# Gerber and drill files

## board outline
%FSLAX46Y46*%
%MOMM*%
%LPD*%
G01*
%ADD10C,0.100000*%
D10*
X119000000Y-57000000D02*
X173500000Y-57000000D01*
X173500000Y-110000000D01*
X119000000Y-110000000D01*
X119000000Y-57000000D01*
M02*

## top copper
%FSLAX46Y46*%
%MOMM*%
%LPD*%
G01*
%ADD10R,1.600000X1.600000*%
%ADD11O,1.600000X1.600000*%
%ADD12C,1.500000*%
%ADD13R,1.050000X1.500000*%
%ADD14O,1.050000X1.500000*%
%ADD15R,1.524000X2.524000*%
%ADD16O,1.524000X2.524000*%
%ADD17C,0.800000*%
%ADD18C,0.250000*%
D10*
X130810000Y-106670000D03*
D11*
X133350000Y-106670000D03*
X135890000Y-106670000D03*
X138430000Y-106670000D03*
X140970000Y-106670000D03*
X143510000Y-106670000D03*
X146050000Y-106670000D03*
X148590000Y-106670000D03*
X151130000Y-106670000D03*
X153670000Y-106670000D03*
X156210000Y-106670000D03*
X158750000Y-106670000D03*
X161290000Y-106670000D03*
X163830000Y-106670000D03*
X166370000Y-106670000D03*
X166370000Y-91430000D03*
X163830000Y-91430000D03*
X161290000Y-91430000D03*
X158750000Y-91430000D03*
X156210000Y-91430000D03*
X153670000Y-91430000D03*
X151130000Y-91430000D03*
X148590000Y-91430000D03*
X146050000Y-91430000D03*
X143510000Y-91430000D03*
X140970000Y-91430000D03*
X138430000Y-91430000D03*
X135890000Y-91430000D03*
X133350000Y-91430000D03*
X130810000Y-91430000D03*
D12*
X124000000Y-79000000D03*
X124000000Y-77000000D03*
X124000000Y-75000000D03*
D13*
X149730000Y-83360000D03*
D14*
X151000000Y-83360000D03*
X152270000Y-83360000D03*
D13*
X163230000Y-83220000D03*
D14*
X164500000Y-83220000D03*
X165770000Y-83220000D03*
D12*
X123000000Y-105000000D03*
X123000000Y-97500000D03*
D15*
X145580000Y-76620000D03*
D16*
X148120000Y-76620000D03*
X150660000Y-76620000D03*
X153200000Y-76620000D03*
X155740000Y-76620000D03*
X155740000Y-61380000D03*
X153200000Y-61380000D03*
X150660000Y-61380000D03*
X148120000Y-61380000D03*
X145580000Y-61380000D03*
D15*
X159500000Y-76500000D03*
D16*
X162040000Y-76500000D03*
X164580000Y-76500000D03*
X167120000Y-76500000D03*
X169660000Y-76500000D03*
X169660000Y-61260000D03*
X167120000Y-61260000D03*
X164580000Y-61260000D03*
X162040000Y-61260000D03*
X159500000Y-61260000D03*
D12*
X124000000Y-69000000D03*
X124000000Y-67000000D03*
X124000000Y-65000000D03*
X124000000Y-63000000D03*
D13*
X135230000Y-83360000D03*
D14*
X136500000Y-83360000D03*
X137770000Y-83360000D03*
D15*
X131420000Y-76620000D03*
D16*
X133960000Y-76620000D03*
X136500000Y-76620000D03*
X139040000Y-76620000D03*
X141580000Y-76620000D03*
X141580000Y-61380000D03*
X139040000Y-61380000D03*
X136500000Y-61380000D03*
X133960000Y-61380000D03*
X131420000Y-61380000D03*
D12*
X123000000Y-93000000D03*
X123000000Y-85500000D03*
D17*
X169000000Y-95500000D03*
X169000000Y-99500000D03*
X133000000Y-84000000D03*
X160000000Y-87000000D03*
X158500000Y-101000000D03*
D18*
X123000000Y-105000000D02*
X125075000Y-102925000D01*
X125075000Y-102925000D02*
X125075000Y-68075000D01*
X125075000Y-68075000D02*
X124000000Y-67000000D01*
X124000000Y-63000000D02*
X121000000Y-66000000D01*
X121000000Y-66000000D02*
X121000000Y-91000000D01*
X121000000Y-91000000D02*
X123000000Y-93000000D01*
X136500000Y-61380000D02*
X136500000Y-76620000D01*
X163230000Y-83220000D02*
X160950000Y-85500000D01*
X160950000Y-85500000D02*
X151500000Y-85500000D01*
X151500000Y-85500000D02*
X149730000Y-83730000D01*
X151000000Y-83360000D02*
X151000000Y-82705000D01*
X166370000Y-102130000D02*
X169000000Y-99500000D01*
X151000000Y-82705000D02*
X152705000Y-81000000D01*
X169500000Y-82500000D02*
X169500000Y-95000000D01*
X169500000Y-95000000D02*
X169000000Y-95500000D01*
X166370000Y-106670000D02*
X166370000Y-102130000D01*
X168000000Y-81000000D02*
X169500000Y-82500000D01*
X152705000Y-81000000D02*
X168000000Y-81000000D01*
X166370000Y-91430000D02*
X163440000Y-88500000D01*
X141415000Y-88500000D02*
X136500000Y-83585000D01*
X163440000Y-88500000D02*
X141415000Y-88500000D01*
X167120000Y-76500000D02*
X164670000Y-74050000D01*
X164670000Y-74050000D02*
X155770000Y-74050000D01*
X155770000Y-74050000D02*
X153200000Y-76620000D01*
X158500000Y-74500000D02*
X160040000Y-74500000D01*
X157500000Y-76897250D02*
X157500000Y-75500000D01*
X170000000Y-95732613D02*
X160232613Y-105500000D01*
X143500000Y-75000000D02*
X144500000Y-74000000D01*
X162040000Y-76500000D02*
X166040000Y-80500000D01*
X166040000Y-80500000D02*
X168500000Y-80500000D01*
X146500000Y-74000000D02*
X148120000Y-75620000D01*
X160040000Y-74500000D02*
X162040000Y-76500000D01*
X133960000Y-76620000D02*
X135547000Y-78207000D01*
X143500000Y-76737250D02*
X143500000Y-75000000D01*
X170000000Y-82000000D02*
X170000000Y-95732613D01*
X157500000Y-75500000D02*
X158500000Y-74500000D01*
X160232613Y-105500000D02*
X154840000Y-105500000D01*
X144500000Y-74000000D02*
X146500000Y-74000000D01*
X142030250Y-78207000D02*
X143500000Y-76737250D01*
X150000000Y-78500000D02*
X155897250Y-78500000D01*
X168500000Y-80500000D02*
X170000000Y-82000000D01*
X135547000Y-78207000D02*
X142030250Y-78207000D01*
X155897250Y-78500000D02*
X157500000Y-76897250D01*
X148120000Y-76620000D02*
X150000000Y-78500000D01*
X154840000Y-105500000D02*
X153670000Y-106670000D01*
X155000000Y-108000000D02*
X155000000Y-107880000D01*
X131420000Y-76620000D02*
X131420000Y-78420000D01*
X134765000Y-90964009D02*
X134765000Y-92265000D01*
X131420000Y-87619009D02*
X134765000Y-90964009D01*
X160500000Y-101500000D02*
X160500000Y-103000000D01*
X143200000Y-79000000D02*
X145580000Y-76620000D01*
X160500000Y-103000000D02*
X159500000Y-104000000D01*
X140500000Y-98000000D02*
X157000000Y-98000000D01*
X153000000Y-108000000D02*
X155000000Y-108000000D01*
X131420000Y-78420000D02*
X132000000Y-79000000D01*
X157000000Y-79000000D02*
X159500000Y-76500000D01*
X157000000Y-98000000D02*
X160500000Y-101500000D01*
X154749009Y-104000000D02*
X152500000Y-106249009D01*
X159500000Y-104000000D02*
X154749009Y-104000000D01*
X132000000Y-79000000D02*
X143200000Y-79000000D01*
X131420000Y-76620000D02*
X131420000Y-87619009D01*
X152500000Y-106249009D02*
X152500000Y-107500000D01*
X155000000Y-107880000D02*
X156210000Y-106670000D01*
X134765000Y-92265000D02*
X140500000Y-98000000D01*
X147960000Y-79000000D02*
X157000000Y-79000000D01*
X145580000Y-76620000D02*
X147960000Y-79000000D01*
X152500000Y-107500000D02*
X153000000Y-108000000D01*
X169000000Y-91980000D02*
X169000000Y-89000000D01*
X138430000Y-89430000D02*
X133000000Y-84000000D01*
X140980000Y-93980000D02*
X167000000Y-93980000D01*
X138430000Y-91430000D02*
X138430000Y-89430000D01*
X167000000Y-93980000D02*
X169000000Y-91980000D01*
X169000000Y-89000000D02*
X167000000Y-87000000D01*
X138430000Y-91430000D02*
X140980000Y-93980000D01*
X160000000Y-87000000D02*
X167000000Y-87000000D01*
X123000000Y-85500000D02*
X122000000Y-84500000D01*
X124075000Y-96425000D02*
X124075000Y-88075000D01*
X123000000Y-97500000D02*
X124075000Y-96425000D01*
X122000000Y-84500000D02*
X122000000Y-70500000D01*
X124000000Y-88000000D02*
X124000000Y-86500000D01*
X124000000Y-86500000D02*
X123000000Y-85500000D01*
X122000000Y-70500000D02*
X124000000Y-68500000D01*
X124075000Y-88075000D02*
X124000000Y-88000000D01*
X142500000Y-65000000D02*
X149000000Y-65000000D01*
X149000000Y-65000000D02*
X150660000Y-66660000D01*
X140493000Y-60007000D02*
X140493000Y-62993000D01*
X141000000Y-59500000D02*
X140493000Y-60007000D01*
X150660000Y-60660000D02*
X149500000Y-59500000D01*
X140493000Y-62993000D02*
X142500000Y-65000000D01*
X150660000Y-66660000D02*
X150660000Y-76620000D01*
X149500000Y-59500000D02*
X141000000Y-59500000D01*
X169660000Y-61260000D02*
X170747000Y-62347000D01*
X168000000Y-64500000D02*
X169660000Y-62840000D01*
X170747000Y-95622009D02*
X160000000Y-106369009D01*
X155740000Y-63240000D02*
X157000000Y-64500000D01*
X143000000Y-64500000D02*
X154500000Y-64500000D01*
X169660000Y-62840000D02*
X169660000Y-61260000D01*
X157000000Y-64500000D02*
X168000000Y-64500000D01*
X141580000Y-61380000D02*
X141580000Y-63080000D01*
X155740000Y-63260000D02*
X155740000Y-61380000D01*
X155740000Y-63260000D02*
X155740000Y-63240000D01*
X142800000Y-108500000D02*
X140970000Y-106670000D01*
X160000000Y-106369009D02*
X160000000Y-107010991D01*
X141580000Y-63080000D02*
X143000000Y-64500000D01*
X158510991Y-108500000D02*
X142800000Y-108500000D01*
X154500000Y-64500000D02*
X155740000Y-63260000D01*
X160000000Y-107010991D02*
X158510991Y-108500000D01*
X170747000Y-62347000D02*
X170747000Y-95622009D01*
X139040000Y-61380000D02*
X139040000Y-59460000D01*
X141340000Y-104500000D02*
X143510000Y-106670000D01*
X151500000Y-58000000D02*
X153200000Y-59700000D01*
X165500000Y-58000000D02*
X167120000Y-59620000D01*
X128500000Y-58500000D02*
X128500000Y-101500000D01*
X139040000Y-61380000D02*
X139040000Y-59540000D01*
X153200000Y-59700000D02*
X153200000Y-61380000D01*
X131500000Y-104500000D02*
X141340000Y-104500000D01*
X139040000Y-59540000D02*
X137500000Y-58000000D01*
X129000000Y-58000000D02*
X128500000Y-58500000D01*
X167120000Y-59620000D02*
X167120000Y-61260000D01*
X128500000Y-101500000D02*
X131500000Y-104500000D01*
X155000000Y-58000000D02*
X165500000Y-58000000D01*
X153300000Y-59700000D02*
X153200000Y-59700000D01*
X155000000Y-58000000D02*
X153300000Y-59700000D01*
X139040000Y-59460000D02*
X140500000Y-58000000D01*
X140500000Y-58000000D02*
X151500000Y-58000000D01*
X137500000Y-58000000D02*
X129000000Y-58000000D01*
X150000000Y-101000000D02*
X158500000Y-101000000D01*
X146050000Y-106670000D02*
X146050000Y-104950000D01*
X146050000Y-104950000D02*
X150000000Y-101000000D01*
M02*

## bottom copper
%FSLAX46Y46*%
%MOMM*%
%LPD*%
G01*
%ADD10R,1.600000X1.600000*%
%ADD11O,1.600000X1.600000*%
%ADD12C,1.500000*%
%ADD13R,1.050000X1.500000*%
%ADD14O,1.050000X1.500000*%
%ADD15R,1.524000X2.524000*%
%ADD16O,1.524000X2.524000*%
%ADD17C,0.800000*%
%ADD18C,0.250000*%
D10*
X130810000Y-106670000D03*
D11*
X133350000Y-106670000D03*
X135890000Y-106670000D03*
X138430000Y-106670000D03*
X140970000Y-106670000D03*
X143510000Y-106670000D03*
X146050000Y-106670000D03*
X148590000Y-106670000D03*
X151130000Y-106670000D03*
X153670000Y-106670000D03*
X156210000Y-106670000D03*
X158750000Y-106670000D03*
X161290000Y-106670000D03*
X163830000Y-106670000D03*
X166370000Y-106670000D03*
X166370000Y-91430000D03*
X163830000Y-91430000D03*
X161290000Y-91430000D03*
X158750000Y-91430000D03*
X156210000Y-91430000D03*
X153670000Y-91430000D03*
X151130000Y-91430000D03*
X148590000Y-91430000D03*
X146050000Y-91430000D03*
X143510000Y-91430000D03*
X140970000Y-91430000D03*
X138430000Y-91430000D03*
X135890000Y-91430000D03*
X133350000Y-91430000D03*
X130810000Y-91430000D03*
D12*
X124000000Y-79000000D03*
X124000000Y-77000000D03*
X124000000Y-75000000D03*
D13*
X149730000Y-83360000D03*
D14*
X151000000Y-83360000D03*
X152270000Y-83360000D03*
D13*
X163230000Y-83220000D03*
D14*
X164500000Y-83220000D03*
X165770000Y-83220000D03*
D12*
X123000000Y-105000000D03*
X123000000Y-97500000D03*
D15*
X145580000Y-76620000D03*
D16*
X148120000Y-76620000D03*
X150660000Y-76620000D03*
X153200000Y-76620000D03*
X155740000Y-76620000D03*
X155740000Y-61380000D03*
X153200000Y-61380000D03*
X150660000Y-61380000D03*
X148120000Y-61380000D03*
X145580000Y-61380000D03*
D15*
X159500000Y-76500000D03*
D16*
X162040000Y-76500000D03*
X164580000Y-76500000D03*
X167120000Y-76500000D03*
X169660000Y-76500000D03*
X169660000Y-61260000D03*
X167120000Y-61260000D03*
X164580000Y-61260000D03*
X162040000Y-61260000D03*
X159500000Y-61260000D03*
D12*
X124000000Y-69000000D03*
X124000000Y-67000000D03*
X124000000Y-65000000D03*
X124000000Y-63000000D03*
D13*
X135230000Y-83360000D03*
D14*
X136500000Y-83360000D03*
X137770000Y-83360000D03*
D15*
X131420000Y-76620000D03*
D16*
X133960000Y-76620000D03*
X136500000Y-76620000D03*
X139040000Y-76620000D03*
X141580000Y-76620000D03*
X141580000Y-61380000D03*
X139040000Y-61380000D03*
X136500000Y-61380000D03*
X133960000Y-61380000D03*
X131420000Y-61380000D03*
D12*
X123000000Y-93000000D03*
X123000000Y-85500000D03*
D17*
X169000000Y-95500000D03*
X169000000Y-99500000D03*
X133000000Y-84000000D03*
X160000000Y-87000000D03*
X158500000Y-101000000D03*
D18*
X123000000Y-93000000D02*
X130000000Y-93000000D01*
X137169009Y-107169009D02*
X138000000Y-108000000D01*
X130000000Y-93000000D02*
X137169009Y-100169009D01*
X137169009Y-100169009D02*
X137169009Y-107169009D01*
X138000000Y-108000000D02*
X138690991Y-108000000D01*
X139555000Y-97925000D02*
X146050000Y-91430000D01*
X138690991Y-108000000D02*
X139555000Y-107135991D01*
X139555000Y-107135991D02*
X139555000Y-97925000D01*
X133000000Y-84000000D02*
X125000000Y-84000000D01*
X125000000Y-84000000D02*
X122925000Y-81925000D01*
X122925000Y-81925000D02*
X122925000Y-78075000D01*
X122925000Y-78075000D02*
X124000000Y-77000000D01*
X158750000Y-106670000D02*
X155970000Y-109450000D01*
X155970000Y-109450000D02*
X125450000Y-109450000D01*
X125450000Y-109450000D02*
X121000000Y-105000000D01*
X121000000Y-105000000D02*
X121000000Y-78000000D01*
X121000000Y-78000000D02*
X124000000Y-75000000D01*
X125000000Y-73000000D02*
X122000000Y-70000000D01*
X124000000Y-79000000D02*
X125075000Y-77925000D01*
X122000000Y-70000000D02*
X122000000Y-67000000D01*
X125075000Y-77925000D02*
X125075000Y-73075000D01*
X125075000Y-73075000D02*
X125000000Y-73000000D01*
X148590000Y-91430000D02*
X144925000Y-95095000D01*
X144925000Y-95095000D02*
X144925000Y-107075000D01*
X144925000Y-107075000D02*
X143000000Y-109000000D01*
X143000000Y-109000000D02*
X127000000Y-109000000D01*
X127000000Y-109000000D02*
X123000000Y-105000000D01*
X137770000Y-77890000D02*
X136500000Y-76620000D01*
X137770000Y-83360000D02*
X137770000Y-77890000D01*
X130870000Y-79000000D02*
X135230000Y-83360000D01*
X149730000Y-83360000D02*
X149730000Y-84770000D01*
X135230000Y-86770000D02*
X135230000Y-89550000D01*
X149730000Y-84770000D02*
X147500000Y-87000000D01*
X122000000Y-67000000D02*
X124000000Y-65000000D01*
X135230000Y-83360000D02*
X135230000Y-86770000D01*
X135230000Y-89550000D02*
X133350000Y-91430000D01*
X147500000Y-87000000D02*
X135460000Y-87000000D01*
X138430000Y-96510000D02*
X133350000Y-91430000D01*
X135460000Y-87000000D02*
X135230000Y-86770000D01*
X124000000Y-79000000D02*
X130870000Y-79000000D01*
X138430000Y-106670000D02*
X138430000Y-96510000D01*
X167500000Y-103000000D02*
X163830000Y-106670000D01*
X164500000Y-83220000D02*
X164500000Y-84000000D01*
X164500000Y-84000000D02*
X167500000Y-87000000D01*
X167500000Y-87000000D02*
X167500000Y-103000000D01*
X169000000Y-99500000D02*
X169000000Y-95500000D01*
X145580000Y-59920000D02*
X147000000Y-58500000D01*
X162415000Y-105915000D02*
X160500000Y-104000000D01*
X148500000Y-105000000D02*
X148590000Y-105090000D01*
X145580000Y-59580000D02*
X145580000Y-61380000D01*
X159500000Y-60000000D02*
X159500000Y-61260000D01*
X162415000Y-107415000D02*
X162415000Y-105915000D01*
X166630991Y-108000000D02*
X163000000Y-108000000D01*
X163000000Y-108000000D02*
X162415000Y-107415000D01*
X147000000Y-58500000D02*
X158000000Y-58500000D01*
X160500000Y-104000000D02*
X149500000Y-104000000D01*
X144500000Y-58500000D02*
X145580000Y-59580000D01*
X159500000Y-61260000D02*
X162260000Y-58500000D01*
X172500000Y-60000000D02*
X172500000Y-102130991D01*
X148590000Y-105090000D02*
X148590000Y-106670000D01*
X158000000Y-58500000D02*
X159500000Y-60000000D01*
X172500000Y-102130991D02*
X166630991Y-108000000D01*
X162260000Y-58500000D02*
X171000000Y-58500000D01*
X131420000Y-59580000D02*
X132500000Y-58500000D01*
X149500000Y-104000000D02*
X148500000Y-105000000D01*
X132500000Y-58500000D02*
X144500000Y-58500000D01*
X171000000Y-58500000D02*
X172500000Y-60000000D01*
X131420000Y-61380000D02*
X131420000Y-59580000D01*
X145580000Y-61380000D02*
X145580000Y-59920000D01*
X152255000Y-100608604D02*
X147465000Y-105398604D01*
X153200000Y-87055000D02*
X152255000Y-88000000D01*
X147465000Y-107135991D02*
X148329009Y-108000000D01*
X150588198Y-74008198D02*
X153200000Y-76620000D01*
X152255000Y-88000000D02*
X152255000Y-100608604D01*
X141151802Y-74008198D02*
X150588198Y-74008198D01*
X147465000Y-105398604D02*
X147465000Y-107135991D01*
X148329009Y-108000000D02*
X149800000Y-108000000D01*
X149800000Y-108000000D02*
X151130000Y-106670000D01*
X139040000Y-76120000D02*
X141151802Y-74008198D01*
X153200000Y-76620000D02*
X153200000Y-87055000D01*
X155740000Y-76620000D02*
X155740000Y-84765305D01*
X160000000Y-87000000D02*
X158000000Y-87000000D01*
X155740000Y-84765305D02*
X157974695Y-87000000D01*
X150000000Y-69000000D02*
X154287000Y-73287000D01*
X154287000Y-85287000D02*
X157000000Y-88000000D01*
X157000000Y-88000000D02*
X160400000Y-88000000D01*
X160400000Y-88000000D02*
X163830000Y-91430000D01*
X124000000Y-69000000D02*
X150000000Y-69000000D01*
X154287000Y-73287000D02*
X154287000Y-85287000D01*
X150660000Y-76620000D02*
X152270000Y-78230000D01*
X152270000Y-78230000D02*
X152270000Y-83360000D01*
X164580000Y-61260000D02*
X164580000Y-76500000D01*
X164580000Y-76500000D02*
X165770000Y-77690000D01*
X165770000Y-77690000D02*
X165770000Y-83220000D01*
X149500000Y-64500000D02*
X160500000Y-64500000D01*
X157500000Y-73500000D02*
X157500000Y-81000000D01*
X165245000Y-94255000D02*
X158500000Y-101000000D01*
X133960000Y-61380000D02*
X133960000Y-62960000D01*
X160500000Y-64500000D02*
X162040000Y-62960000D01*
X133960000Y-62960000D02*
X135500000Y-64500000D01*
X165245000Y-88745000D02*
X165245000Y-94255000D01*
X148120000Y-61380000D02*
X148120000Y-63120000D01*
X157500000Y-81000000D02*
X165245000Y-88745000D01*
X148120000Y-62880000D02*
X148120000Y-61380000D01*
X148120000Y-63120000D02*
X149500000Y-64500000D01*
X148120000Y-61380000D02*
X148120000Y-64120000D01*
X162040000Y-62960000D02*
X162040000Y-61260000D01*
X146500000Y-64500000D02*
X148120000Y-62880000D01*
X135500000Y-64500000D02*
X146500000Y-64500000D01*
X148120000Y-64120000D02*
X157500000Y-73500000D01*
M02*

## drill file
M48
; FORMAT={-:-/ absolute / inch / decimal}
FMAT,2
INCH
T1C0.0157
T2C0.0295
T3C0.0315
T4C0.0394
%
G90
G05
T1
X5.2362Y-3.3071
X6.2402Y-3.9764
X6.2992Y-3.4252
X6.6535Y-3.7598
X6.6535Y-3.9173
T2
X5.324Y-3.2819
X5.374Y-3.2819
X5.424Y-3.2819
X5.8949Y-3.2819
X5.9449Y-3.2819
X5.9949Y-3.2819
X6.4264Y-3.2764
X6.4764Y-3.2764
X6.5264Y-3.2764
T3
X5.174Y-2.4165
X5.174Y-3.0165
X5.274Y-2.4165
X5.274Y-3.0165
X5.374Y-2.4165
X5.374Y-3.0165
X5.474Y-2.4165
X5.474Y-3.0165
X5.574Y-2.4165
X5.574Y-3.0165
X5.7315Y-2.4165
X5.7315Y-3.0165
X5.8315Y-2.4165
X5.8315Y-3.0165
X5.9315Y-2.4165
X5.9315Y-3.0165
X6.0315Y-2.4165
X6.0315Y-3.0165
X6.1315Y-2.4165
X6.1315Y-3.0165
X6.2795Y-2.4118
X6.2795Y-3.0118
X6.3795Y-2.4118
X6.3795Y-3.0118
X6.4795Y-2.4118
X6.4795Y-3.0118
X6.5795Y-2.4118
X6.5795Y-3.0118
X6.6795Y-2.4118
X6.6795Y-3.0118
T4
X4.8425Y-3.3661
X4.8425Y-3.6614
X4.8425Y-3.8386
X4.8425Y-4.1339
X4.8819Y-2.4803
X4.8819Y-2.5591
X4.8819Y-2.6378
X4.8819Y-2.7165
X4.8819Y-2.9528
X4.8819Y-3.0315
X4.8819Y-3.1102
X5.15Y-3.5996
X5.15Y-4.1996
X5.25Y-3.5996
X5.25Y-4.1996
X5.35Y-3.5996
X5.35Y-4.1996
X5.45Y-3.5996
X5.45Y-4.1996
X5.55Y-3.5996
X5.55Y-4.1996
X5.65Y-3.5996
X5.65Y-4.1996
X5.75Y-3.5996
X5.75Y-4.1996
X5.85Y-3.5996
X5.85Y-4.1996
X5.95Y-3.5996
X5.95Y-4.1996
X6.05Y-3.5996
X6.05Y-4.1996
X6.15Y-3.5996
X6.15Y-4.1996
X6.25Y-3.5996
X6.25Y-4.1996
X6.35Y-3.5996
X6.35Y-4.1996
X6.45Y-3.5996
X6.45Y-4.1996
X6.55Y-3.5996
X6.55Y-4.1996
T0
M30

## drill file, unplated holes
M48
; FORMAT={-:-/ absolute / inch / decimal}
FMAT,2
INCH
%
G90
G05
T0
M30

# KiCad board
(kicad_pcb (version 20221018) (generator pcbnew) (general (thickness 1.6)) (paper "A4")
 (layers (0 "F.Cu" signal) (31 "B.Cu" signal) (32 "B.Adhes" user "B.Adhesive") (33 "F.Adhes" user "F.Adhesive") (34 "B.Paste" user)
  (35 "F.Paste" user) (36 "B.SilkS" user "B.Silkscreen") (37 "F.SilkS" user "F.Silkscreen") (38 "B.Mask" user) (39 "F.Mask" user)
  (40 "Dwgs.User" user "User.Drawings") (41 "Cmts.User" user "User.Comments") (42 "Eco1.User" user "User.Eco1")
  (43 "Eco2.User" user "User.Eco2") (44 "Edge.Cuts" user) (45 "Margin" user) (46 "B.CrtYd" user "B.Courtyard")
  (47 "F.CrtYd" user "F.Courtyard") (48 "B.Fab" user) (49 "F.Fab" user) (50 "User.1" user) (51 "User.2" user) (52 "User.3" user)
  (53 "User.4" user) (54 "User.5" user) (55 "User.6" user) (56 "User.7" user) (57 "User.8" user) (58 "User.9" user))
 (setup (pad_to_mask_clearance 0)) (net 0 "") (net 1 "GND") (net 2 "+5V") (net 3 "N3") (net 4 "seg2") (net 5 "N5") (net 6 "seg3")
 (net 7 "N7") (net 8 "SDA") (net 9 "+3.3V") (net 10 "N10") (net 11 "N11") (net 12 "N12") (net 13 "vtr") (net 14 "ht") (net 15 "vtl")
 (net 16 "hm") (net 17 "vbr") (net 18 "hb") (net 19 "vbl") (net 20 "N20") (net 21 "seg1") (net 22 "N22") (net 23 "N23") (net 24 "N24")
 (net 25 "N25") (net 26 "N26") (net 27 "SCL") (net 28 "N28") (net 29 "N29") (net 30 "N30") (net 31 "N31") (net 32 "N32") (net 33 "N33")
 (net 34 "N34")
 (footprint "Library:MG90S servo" (layer "F.Cu") (at 124 77 90)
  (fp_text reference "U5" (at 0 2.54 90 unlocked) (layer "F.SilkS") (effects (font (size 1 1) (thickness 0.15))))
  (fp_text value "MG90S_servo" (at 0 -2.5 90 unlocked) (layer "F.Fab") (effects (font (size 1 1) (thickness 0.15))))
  (pad "1" thru_hole circle (at -2 0 90) (size 1.5 1.5) (drill 1) (layers "*.Cu" "*.Mask") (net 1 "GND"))
  (pad "2" thru_hole circle (at 0 0 90) (size 1.5 1.5) (drill 1) (layers "*.Cu" "*.Mask") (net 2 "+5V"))
  (pad "3" thru_hole circle (at 2 0 90) (size 1.5 1.5) (drill 1) (layers "*.Cu" "*.Mask") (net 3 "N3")))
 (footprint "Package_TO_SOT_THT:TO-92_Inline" (layer "F.Cu") (at 149.73 83.36)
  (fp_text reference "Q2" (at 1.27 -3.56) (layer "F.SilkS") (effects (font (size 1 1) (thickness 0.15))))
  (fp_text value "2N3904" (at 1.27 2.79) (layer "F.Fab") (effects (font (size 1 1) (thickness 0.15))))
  (pad "1" thru_hole rect (at 0 0) (size 1.05 1.5) (drill 0.75) (layers "*.Cu" "*.Mask") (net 1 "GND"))
  (pad "2" thru_hole oval (at 1.27 0) (size 1.05 1.5) (drill 0.75) (layers "*.Cu" "*.Mask") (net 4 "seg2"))
  (pad "3" thru_hole oval (at 2.54 0) (size 1.05 1.5) (drill 0.75) (layers "*.Cu" "*.Mask") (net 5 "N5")))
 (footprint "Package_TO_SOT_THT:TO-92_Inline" (layer "F.Cu") (at 163.23 83.22)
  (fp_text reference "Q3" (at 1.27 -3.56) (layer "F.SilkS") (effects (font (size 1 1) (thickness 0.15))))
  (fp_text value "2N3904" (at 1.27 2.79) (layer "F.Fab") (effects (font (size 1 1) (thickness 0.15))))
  (pad "1" thru_hole rect (at 0 0) (size 1.05 1.5) (drill 0.75) (layers "*.Cu" "*.Mask") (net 1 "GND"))
  (pad "2" thru_hole oval (at 1.27 0) (size 1.05 1.5) (drill 0.75) (layers "*.Cu" "*.Mask") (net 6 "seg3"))
  (pad "3" thru_hole oval (at 2.54 0) (size 1.05 1.5) (drill 0.75) (layers "*.Cu" "*.Mask") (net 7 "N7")))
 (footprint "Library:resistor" (layer "F.Cu") (at 123 105 90)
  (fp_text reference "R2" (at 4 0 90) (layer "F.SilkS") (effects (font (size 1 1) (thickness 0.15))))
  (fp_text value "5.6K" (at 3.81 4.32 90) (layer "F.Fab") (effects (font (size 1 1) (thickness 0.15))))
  (pad "1" thru_hole circle (at 0 0 90) (size 1.5 1.5) (drill 1) (layers "*.Cu" "*.Mask") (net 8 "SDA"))
  (pad "2" thru_hole circle (at 7.5 0 90) (size 1.5 1.5) (drill 1) (layers "*.Cu" "*.Mask") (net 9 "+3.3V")))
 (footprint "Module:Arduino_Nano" (layer "F.Cu") (at 130.81 106.67 90)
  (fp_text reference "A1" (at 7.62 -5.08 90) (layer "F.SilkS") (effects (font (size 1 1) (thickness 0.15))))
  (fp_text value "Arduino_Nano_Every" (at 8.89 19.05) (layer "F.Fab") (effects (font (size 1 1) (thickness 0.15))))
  (pad "1" thru_hole rect (at 0 0 90) (size 1.6 1.6) (drill 1) (layers "*.Cu" "*.Mask") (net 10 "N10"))
  (pad "2" thru_hole oval (at 0 2.54 90) (size 1.6 1.6) (drill 1) (layers "*.Cu" "*.Mask") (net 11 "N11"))
  (pad "3" thru_hole oval (at 0 5.08 90) (size 1.6 1.6) (drill 1) (layers "*.Cu" "*.Mask") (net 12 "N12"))
  (pad "4" thru_hole oval (at 0 7.62 90) (size 1.6 1.6) (drill 1) (layers "*.Cu" "*.Mask") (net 1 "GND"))
  (pad "5" thru_hole oval (at 0 10.16 90) (size 1.6 1.6) (drill 1) (layers "*.Cu" "*.Mask") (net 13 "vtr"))
  (pad "6" thru_hole oval (at 0 12.7 90) (size 1.6 1.6) (drill 1) (layers "*.Cu" "*.Mask") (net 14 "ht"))
  (pad "7" thru_hole oval (at 0 15.24 90) (size 1.6 1.6) (drill 1) (layers "*.Cu" "*.Mask") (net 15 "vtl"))
  (pad "8" thru_hole oval (at 0 17.78 90) (size 1.6 1.6) (drill 1) (layers "*.Cu" "*.Mask") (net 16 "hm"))
  (pad "9" thru_hole oval (at 0 20.32 90) (size 1.6 1.6) (drill 1) (layers "*.Cu" "*.Mask") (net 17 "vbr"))
  (pad "10" thru_hole oval (at 0 22.86 90) (size 1.6 1.6) (drill 1) (layers "*.Cu" "*.Mask") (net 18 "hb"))
  (pad "11" thru_hole oval (at 0 25.4 90) (size 1.6 1.6) (drill 1) (layers "*.Cu" "*.Mask") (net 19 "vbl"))
  (pad "12" thru_hole oval (at 0 27.94 90) (size 1.6 1.6) (drill 1) (layers "*.Cu" "*.Mask") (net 3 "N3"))
  (pad "13" thru_hole oval (at 0 30.48 90) (size 1.6 1.6) (drill 1) (layers "*.Cu" "*.Mask") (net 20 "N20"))
  (pad "14" thru_hole oval (at 0 33.02 90) (size 1.6 1.6) (drill 1) (layers "*.Cu" "*.Mask") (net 6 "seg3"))
  (pad "15" thru_hole oval (at 0 35.56 90) (size 1.6 1.6) (drill 1) (layers "*.Cu" "*.Mask") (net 4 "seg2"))
  (pad "16" thru_hole oval (at 15.24 35.56 90) (size 1.6 1.6) (drill 1) (layers "*.Cu" "*.Mask") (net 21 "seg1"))
  (pad "17" thru_hole oval (at 15.24 33.02 90) (size 1.6 1.6) (drill 1) (layers "*.Cu" "*.Mask") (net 9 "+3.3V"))
  (pad "18" thru_hole oval (at 15.24 30.48 90) (size 1.6 1.6) (drill 1) (layers "*.Cu" "*.Mask") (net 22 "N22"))
  (pad "19" thru_hole oval (at 15.24 27.94 90) (size 1.6 1.6) (drill 1) (layers "*.Cu" "*.Mask") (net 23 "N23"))
  (pad "20" thru_hole oval (at 15.24 25.4 90) (size 1.6 1.6) (drill 1) (layers "*.Cu" "*.Mask") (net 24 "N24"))
  (pad "21" thru_hole oval (at 15.24 22.86 90) (size 1.6 1.6) (drill 1) (layers "*.Cu" "*.Mask") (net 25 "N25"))
  (pad "22" thru_hole oval (at 15.24 20.32 90) (size 1.6 1.6) (drill 1) (layers "*.Cu" "*.Mask") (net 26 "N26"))
  (pad "23" thru_hole oval (at 15.24 17.78 90) (size 1.6 1.6) (drill 1) (layers "*.Cu" "*.Mask") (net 8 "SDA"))
  (pad "24" thru_hole oval (at 15.24 15.24 90) (size 1.6 1.6) (drill 1) (layers "*.Cu" "*.Mask") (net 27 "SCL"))
  (pad "25" thru_hole oval (at 15.24 12.7 90) (size 1.6 1.6) (drill 1) (layers "*.Cu" "*.Mask") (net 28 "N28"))
  (pad "26" thru_hole oval (at 15.24 10.16 90) (size 1.6 1.6) (drill 1) (layers "*.Cu" "*.Mask") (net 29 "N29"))
  (pad "27" thru_hole oval (at 15.24 7.62 90) (size 1.6 1.6) (drill 1) (layers "*.Cu" "*.Mask") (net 2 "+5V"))
  (pad "28" thru_hole oval (at 15.24 5.08 90) (size 1.6 1.6) (drill 1) (layers "*.Cu" "*.Mask") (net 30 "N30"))
  (pad "29" thru_hole oval (at 15.24 2.54 90) (size 1.6 1.6) (drill 1) (layers "*.Cu" "*.Mask") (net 1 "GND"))
  (pad "30" thru_hole oval (at 15.24 0 90) (size 1.6 1.6) (drill 1) (layers "*.Cu" "*.Mask") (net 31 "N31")))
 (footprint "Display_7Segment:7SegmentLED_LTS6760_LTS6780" (layer "F.Cu") (at 145.58 76.62 90)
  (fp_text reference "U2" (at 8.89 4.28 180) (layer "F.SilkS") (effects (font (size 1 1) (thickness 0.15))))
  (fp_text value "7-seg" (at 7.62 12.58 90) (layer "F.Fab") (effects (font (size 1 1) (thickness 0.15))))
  (pad "1" thru_hole rect (at 0 0) (size 1.524 2.524) (drill 0.8) (layers "*.Cu" "*.Mask") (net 19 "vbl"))
  (pad "2" thru_hole oval (at 0 2.54) (size 1.524 2.524) (drill 0.8) (layers "*.Cu" "*.Mask") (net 18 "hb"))
  (pad "3" thru_hole oval (at 0 5.08) (size 1.524 2.524) (drill 0.8) (layers "*.Cu" "*.Mask") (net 5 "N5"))
  (pad "4" thru_hole oval (at 0 7.62) (size 1.524 2.524) (drill 0.8) (layers "*.Cu" "*.Mask") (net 17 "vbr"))
  (pad "5" thru_hole oval (at 0 10.16) (size 1.524 2.524) (drill 0.8) (layers "*.Cu" "*.Mask") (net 2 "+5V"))
  (pad "6" thru_hole oval (at 15.24 10.16) (size 1.524 2.524) (drill 0.8) (layers "*.Cu" "*.Mask") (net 13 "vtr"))
  (pad "7" thru_hole oval (at 15.24 7.62) (size 1.524 2.524) (drill 0.8) (layers "*.Cu" "*.Mask") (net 14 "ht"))
  (pad "8" thru_hole oval (at 15.24 5.08) (size 1.524 2.524) (drill 0.8) (layers "*.Cu" "*.Mask") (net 5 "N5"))
  (pad "9" thru_hole oval (at 15.24 2.54) (size 1.524 2.524) (drill 0.8) (layers "*.Cu" "*.Mask") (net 15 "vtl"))
  (pad "10" thru_hole oval (at 15.24 0) (size 1.524 2.524) (drill 0.8) (layers "*.Cu" "*.Mask") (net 16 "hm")))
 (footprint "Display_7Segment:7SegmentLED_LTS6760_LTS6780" (layer "F.Cu") (at 159.5 76.5 90)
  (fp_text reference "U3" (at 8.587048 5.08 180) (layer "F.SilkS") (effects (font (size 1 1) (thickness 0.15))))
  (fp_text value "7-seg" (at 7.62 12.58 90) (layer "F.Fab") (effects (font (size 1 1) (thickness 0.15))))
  (pad "1" thru_hole rect (at 0 0) (size 1.524 2.524) (drill 0.8) (layers "*.Cu" "*.Mask") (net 19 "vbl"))
  (pad "2" thru_hole oval (at 0 2.54) (size 1.524 2.524) (drill 0.8) (layers "*.Cu" "*.Mask") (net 18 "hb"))
  (pad "3" thru_hole oval (at 0 5.08) (size 1.524 2.524) (drill 0.8) (layers "*.Cu" "*.Mask") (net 7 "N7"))
  (pad "4" thru_hole oval (at 0 7.62) (size 1.524 2.524) (drill 0.8) (layers "*.Cu" "*.Mask") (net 17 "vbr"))
  (pad "5" thru_hole oval (at 0 10.16) (size 1.524 2.524) (drill 0.8) (layers "*.Cu" "*.Mask") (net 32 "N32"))
  (pad "6" thru_hole oval (at 15.24 10.16) (size 1.524 2.524) (drill 0.8) (layers "*.Cu" "*.Mask") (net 13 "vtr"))
  (pad "7" thru_hole oval (at 15.24 7.62) (size 1.524 2.524) (drill 0.8) (layers "*.Cu" "*.Mask") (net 14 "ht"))
  (pad "8" thru_hole oval (at 15.24 5.08) (size 1.524 2.524) (drill 0.8) (layers "*.Cu" "*.Mask") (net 7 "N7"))
  (pad "9" thru_hole oval (at 15.24 2.54) (size 1.524 2.524) (drill 0.8) (layers "*.Cu" "*.Mask") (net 15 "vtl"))
  (pad "10" thru_hole oval (at 15.24 0) (size 1.524 2.524) (drill 0.8) (layers "*.Cu" "*.Mask") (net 16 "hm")))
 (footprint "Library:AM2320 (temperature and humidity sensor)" (layer "F.Cu") (at 124 66 90)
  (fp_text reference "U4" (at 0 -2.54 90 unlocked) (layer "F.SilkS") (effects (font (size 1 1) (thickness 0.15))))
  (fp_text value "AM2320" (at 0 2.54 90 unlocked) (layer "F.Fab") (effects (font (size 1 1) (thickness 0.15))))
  (pad "1" thru_hole circle (at -3 0 90) (size 1.5 1.5) (drill 1) (layers "*.Cu" "*.Mask") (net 9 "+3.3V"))
  (pad "2" thru_hole circle (at -1 0 90) (size 1.5 1.5) (drill 1) (layers "*.Cu" "*.Mask") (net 8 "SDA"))
  (pad "3" thru_hole circle (at 1 0 90) (size 1.5 1.5) (drill 1) (layers "*.Cu" "*.Mask") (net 1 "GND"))
  (pad "4" thru_hole circle (at 3 0 90) (size 1.5 1.5) (drill 1) (layers "*.Cu" "*.Mask") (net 27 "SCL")))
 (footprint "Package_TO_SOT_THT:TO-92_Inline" (layer "F.Cu") (at 135.23 83.36)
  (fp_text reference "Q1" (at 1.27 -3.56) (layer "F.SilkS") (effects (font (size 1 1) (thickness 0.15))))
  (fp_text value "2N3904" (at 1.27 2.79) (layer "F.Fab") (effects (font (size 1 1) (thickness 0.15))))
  (pad "1" thru_hole rect (at 0 0) (size 1.05 1.5) (drill 0.75) (layers "*.Cu" "*.Mask") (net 1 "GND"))
  (pad "2" thru_hole oval (at 1.27 0) (size 1.05 1.5) (drill 0.75) (layers "*.Cu" "*.Mask") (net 21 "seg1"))
  (pad "3" thru_hole oval (at 2.54 0) (size 1.05 1.5) (drill 0.75) (layers "*.Cu" "*.Mask") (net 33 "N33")))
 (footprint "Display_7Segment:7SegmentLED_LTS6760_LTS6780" (layer "F.Cu") (at 131.42 76.62 90)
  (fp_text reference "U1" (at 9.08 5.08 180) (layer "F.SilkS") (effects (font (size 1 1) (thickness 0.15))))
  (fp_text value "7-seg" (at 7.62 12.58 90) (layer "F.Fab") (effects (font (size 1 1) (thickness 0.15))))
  (pad "1" thru_hole rect (at 0 0) (size 1.524 2.524) (drill 0.8) (layers "*.Cu" "*.Mask") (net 19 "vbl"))
  (pad "2" thru_hole oval (at 0 2.54) (size 1.524 2.524) (drill 0.8) (layers "*.Cu" "*.Mask") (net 18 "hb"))
  (pad "3" thru_hole oval (at 0 5.08) (size 1.524 2.524) (drill 0.8) (layers "*.Cu" "*.Mask") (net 33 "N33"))
  (pad "4" thru_hole oval (at 0 7.62) (size 1.524 2.524) (drill 0.8) (layers "*.Cu" "*.Mask") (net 17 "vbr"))
  (pad "5" thru_hole oval (at 0 10.16) (size 1.524 2.524) (drill 0.8) (layers "*.Cu" "*.Mask") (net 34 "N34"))
  (pad "6" thru_hole oval (at 15.24 10.16) (size 1.524 2.524) (drill 0.8) (layers "*.Cu" "*.Mask") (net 13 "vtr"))
  (pad "7" thru_hole oval (at 15.24 7.62) (size 1.524 2.524) (drill 0.8) (layers "*.Cu" "*.Mask") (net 14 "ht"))
  (pad "8" thru_hole oval (at 15.24 5.08) (size 1.524 2.524) (drill 0.8) (layers "*.Cu" "*.Mask") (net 33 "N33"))
  (pad "9" thru_hole oval (at 15.24 2.54) (size 1.524 2.524) (drill 0.8) (layers "*.Cu" "*.Mask") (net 15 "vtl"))
  (pad "10" thru_hole oval (at 15.24 0) (size 1.524 2.524) (drill 0.8) (layers "*.Cu" "*.Mask") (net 16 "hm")))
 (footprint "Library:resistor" (layer "F.Cu") (at 123 93 90)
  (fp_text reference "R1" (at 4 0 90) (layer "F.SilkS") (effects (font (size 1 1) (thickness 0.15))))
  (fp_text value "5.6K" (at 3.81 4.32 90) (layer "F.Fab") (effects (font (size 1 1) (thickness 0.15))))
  (pad "1" thru_hole circle (at 0 0 90) (size 1.5 1.5) (drill 1) (layers "*.Cu" "*.Mask") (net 27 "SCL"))
  (pad "2" thru_hole circle (at 7.5 0 90) (size 1.5 1.5) (drill 1) (layers "*.Cu" "*.Mask") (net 9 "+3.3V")))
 (gr_rect (start 119 57) (end 173.5 110) (stroke (width 0.1) (type solid)) (fill none) (layer "Edge.Cuts"))
 (segment (start 121 78) (end 124 75) (width 0.25) (layer "B.Cu") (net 3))
 (segment (start 155.97 109.45) (end 125.45 109.45) (width 0.25) (layer "B.Cu") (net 3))
 (segment (start 158.75 106.67) (end 155.97 109.45) (width 0.25) (layer "B.Cu") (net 3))
 (segment (start 121 105) (end 121 78) (width 0.25) (layer "B.Cu") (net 3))
 (segment (start 125.45 109.45) (end 121 105) (width 0.25) (layer "B.Cu") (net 3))
 (segment (start 123 105) (end 125.075 102.925) (width 0.25) (layer "F.Cu") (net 8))
 (segment (start 125.075 102.925) (end 125.075 68.075) (width 0.25) (layer "F.Cu") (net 8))
 (segment (start 125.075 68.075) (end 124 67) (width 0.25) (layer "F.Cu") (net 8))
 (segment (start 144.925 95.095) (end 144.925 107.075) (width 0.25) (layer "B.Cu") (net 8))
 (segment (start 127 109) (end 123 105) (width 0.25) (layer "B.Cu") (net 8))
 (segment (start 144.925 107.075) (end 143 109) (width 0.25) (layer "B.Cu") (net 8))
 (segment (start 143 109) (end 127 109) (width 0.25) (layer "B.Cu") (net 8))
 (segment (start 148.59 91.43) (end 144.925 95.095) (width 0.25) (layer "B.Cu") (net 8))
 (segment (start 124 63) (end 121 66) (width 0.25) (layer "F.Cu") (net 27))
 (segment (start 121 91) (end 123 93) (width 0.25) (layer "F.Cu") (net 27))
 (segment (start 121 66) (end 121 91) (width 0.25) (layer "F.Cu") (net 27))
 (segment (start 139.555 97.925) (end 146.05 91.43) (width 0.25) (layer "B.Cu") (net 27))
 (segment (start 138 108) (end 138.690991 108) (width 0.25) (layer "B.Cu") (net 27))
 (segment (start 123 93) (end 130 93) (width 0.25) (layer "B.Cu") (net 27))
 (segment (start 139.555 107.135991) (end 139.555 97.925) (width 0.25) (layer "B.Cu") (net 27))
 (segment (start 137.169009 100.169009) (end 137.169009 107.169009) (width 0.25) (layer "B.Cu") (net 27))
 (segment (start 138.690991 108) (end 139.555 107.135991) (width 0.25) (layer "B.Cu") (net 27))
 (segment (start 137.169009 107.169009) (end 138 108) (width 0.25) (layer "B.Cu") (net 27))
 (segment (start 130 93) (end 137.169009 100.169009) (width 0.25) (layer "B.Cu") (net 27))
 (segment (start 136.5 61.38) (end 136.5 76.62) (width 0.25) (layer "F.Cu") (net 33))
 (segment (start 137.77 77.89) (end 136.5 76.62) (width 0.25) (layer "B.Cu") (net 33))
 (segment (start 137.77 83.36) (end 137.77 77.89) (width 0.25) (layer "B.Cu") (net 33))
 (segment (start 163.23 83.22) (end 160.95 85.5) (width 0.25) (layer "F.Cu") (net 1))
 (segment (start 160.95 85.5) (end 151.5 85.5) (width 0.25) (layer "F.Cu") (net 1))
 (segment (start 151.5 85.5) (end 149.73 83.73) (width 0.25) (layer "F.Cu") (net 1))
 (segment (start 130.87 79) (end 135.23 83.36) (width 0.25) (layer "B.Cu") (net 1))
 (segment (start 149.73 83.36) (end 149.73 84.77) (width 0.25) (layer "B.Cu") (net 1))
 (segment (start 135.23 86.77) (end 135.23 89.55) (width 0.25) (layer "B.Cu") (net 1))
 (segment (start 125 73) (end 122 70) (width 0.25) (layer "B.Cu") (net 1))
 (segment (start 124 79) (end 125.075 77.925) (width 0.25) (layer "B.Cu") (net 1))
 (segment (start 149.73 84.77) (end 147.5 87) (width 0.25) (layer "B.Cu") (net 1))
 (segment (start 125.075 73.075) (end 125 73) (width 0.25) (layer "B.Cu") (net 1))
 (segment (start 122 70) (end 122 67) (width 0.25) (layer "B.Cu") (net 1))
 (segment (start 122 67) (end 124 65) (width 0.25) (layer "B.Cu") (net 1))
 (segment (start 135.23 83.36) (end 135.23 86.77) (width 0.25) (layer "B.Cu") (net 1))
 (segment (start 135.23 89.55) (end 133.35 91.43) (width 0.25) (layer "B.Cu") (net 1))
 (segment (start 147.5 87) (end 135.46 87) (width 0.25) (layer "B.Cu") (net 1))
 (segment (start 138.43 96.51) (end 133.35 91.43) (width 0.25) (layer "B.Cu") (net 1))
 (segment (start 135.46 87) (end 135.23 86.77) (width 0.25) (layer "B.Cu") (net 1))
 (segment (start 125.075 77.925) (end 125.075 73.075) (width 0.25) (layer "B.Cu") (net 1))
 (segment (start 124 79) (end 130.87 79) (width 0.25) (layer "B.Cu") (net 1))
 (segment (start 138.43 106.67) (end 138.43 96.51) (width 0.25) (layer "B.Cu") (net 1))
 (segment (start 167.5 103) (end 163.83 106.67) (width 0.25) (layer "B.Cu") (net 6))
 (segment (start 164.5 83.22) (end 164.5 84) (width 0.25) (layer "B.Cu") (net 6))
 (segment (start 164.5 84) (end 167.5 87) (width 0.25) (layer "B.Cu") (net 6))
 (segment (start 167.5 87) (end 167.5 103) (width 0.25) (layer "B.Cu") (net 6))
 (segment (start 151 83.36) (end 151 82.705) (width 0.25) (layer "F.Cu") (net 4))
 (segment (start 166.37 102.13) (end 169 99.5) (width 0.25) (layer "F.Cu") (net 4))
 (segment (start 151 82.705) (end 152.705 81) (width 0.25) (layer "F.Cu") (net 4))
 (segment (start 169.5 82.5) (end 169.5 95) (width 0.25) (layer "F.Cu") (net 4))
 (segment (start 169.5 95) (end 169 95.5) (width 0.25) (layer "F.Cu") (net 4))
 (segment (start 166.37 106.67) (end 166.37 102.13) (width 0.25) (layer "F.Cu") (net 4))
 (segment (start 168 81) (end 169.5 82.5) (width 0.25) (layer "F.Cu") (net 4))
 (segment (start 152.705 81) (end 168 81) (width 0.25) (layer "F.Cu") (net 4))
 (via (at 169 95.5) (size 0.8) (drill 0.4) (layers "F.Cu" "B.Cu") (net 4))
 (via (at 169 99.5) (size 0.8) (drill 0.4) (layers "F.Cu" "B.Cu") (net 4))
 (segment (start 169 99.5) (end 169 95.5) (width 0.25) (layer "B.Cu") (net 4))
 (segment (start 166.37 91.43) (end 163.44 88.5) (width 0.25) (layer "F.Cu") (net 21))
 (segment (start 141.415 88.5) (end 136.5 83.585) (width 0.25) (layer "F.Cu") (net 21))
 (segment (start 163.44 88.5) (end 141.415 88.5) (width 0.25) (layer "F.Cu") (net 21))
 (segment (start 145.58 59.92) (end 147 58.5) (width 0.25) (layer "B.Cu") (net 16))
 (segment (start 162.415 105.915) (end 160.5 104) (width 0.25) (layer "B.Cu") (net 16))
 (segment (start 148.5 105) (end 148.59 105.09) (width 0.25) (layer "B.Cu") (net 16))
 (segment (start 145.58 59.58) (end 145.58 61.38) (width 0.25) (layer "B.Cu") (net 16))
 (segment (start 159.5 60) (end 159.5 61.26) (width 0.25) (layer "B.Cu") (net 16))
 (segment (start 162.415 107.415) (end 162.415 105.915) (width 0.25) (layer "B.Cu") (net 16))
 (segment (start 166.630991 108) (end 163 108) (width 0.25) (layer "B.Cu") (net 16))
 (segment (start 163 108) (end 162.415 107.415) (width 0.25) (layer "B.Cu") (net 16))
 (segment (start 147 58.5) (end 158 58.5) (width 0.25) (layer "B.Cu") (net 16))
 (segment (start 160.5 104) (end 149.5 104) (width 0.25) (layer "B.Cu") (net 16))
 (segment (start 144.5 58.5) (end 145.58 59.58) (width 0.25) (layer "B.Cu") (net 16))
 (segment (start 159.5 61.26) (end 162.26 58.5) (width 0.25) (layer "B.Cu") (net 16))
 (segment (start 172.5 60) (end 172.5 102.130991) (width 0.25) (layer "B.Cu") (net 16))
 (segment (start 148.59 105.09) (end 148.59 106.67) (width 0.25) (layer "B.Cu") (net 16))
 (segment (start 158 58.5) (end 159.5 60) (width 0.25) (layer "B.Cu") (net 16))
 (segment (start 172.5 102.130991) (end 166.630991 108) (width 0.25) (layer "B.Cu") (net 16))
 (segment (start 162.26 58.5) (end 171 58.5) (width 0.25) (layer "B.Cu") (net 16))
 (segment (start 131.42 59.58) (end 132.5 58.5) (width 0.25) (layer "B.Cu") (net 16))
 (segment (start 149.5 104) (end 148.5 105) (width 0.25) (layer "B.Cu") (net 16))
 (segment (start 132.5 58.5) (end 144.5 58.5) (width 0.25) (layer "B.Cu") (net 16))
 (segment (start 171 58.5) (end 172.5 60) (width 0.25) (layer "B.Cu") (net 16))
 (segment (start 131.42 61.38) (end 131.42 59.58) (width 0.25) (layer "B.Cu") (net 16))
 (segment (start 145.58 61.38) (end 145.58 59.92) (width 0.25) (layer "B.Cu") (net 16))
 (segment (start 167.12 76.5) (end 164.67 74.05) (width 0.25) (layer "F.Cu") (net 17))
 (segment (start 164.67 74.05) (end 155.77 74.05) (width 0.25) (layer "F.Cu") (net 17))
 (segment (start 155.77 74.05) (end 153.2 76.62) (width 0.25) (layer "F.Cu") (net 17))
 (segment (start 152.255 100.608604) (end 147.465 105.398604) (width 0.25) (layer "B.Cu") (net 17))
 (segment (start 153.2 87.055) (end 152.255 88) (width 0.25) (layer "B.Cu") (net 17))
 (segment (start 147.465 107.135991) (end 148.329009 108) (width 0.25) (layer "B.Cu") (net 17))
 (segment (start 150.588198 74.008198) (end 153.2 76.62) (width 0.25) (layer "B.Cu") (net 17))
 (segment (start 152.255 88) (end 152.255 100.608604) (width 0.25) (layer "B.Cu") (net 17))
 (segment (start 141.151802 74.008198) (end 150.588198 74.008198) (width 0.25) (layer "B.Cu") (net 17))
 (segment (start 147.465 105.398604) (end 147.465 107.135991) (width 0.25) (layer "B.Cu") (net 17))
 (segment (start 148.329009 108) (end 149.8 108) (width 0.25) (layer "B.Cu") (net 17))
 (segment (start 149.8 108) (end 151.13 106.67) (width 0.25) (layer "B.Cu") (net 17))
 (segment (start 139.04 76.12) (end 141.151802 74.008198) (width 0.25) (layer "B.Cu") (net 17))
 (segment (start 153.2 76.62) (end 153.2 87.055) (width 0.25) (layer "B.Cu") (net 17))
 (segment (start 158.5 74.5) (end 160.04 74.5) (width 0.25) (layer "F.Cu") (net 18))
 (segment (start 157.5 76.89725) (end 157.5 75.5) (width 0.25) (layer "F.Cu") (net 18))
 (segment (start 170 95.732613) (end 160.232613 105.5) (width 0.25) (layer "F.Cu") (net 18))
 (segment (start 143.5 75) (end 144.5 74) (width 0.25) (layer "F.Cu") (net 18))
 (segment (start 162.04 76.5) (end 166.04 80.5) (width 0.25) (layer "F.Cu") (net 18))
 (segment (start 166.04 80.5) (end 168.5 80.5) (width 0.25) (layer "F.Cu") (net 18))
 (segment (start 146.5 74) (end 148.12 75.62) (width 0.25) (layer "F.Cu") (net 18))
 (segment (start 160.04 74.5) (end 162.04 76.5) (width 0.25) (layer "F.Cu") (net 18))
 (segment (start 133.96 76.62) (end 135.547 78.207) (width 0.25) (layer "F.Cu") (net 18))
 (segment (start 143.5 76.73725) (end 143.5 75) (width 0.25) (layer "F.Cu") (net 18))
 (segment (start 170 82) (end 170 95.732613) (width 0.25) (layer "F.Cu") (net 18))
 (segment (start 157.5 75.5) (end 158.5 74.5) (width 0.25) (layer "F.Cu") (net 18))
 (segment (start 160.232613 105.5) (end 154.84 105.5) (width 0.25) (layer "F.Cu") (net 18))
 (segment (start 144.5 74) (end 146.5 74) (width 0.25) (layer "F.Cu") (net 18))
 (segment (start 142.03025 78.207) (end 143.5 76.73725) (width 0.25) (layer "F.Cu") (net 18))
 (segment (start 150 78.5) (end 155.89725 78.5) (width 0.25) (layer "F.Cu") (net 18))
 (segment (start 168.5 80.5) (end 170 82) (width 0.25) (layer "F.Cu") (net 18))
 (segment (start 135.547 78.207) (end 142.03025 78.207) (width 0.25) (layer "F.Cu") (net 18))
 (segment (start 155.89725 78.5) (end 157.5 76.89725) (width 0.25) (layer "F.Cu") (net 18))
 (segment (start 148.12 76.62) (end 150 78.5) (width 0.25) (layer "F.Cu") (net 18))
 (segment (start 154.84 105.5) (end 153.67 106.67) (width 0.25) (layer "F.Cu") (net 18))
 (segment (start 155 108) (end 155 107.88) (width 0.25) (layer "F.Cu") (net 19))
 (segment (start 131.42 76.62) (end 131.42 78.42) (width 0.25) (layer "F.Cu") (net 19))
 (segment (start 134.765 90.964009) (end 134.765 92.265) (width 0.25) (layer "F.Cu") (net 19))
 (segment (start 131.42 87.619009) (end 134.765 90.964009) (width 0.25) (layer "F.Cu") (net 19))
 (segment (start 160.5 101.5) (end 160.5 103) (width 0.25) (layer "F.Cu") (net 19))
 (segment (start 143.2 79) (end 145.58 76.62) (width 0.25) (layer "F.Cu") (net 19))
 (segment (start 160.5 103) (end 159.5 104) (width 0.25) (layer "F.Cu") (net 19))
 (segment (start 140.5 98) (end 157 98) (width 0.25) (layer "F.Cu") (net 19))
 (segment (start 153 108) (end 155 108) (width 0.25) (layer "F.Cu") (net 19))
 (segment (start 131.42 78.42) (end 132 79) (width 0.25) (layer "F.Cu") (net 19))
 (segment (start 157 79) (end 159.5 76.5) (width 0.25) (layer "F.Cu") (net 19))
 (segment (start 157 98) (end 160.5 101.5) (width 0.25) (layer "F.Cu") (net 19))
 (segment (start 154.749009 104) (end 152.5 106.249009) (width 0.25) (layer "F.Cu") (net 19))
 (segment (start 159.5 104) (end 154.749009 104) (width 0.25) (layer "F.Cu") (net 19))
 (segment (start 132 79) (end 143.2 79) (width 0.25) (layer "F.Cu") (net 19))
 (segment (start 131.42 76.62) (end 131.42 87.619009) (width 0.25) (layer "F.Cu") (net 19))
 (segment (start 152.5 106.249009) (end 152.5 107.5) (width 0.25) (layer "F.Cu") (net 19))
 (segment (start 155 107.88) (end 156.21 106.67) (width 0.25) (layer "F.Cu") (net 19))
 (segment (start 134.765 92.265) (end 140.5 98) (width 0.25) (layer "F.Cu") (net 19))
 (segment (start 147.96 79) (end 157 79) (width 0.25) (layer "F.Cu") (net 19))
 (segment (start 145.58 76.62) (end 147.96 79) (width 0.25) (layer "F.Cu") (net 19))
 (segment (start 152.5 107.5) (end 153 108) (width 0.25) (layer "F.Cu") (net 19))
 (segment (start 169 91.98) (end 169 89) (width 0.25) (layer "F.Cu") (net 2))
 (segment (start 138.43 89.43) (end 133 84) (width 0.25) (layer "F.Cu") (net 2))
 (segment (start 140.98 93.98) (end 167 93.98) (width 0.25) (layer "F.Cu") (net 2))
 (segment (start 138.43 91.43) (end 138.43 89.43) (width 0.25) (layer "F.Cu") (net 2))
 (segment (start 167 93.98) (end 169 91.98) (width 0.25) (layer "F.Cu") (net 2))
 (segment (start 169 89) (end 167 87) (width 0.25) (layer "F.Cu") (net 2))
 (segment (start 138.43 91.43) (end 140.98 93.98) (width 0.25) (layer "F.Cu") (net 2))
 (segment (start 160 87) (end 167 87) (width 0.25) (layer "F.Cu") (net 2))
 (via (at 133 84) (size 0.8) (drill 0.4) (layers "F.Cu" "B.Cu") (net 2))
 (via (at 160 87) (size 0.8) (drill 0.4) (layers "F.Cu" "B.Cu") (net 2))
 (segment (start 122.925 81.925) (end 122.925 78.075) (width 0.25) (layer "B.Cu") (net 2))
 (segment (start 122.925 78.075) (end 124 77) (width 0.25) (layer "B.Cu") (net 2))
 (segment (start 155.74 76.62) (end 155.74 84.765305) (width 0.25) (layer "B.Cu") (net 2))
 (segment (start 133 84) (end 125 84) (width 0.25) (layer "B.Cu") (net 2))
 (segment (start 125 84) (end 122.925 81.925) (width 0.25) (layer "B.Cu") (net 2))
 (segment (start 160 87) (end 158 87) (width 0.25) (layer "B.Cu") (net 2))
 (segment (start 155.74 84.765305) (end 157.974695 87) (width 0.25) (layer "B.Cu") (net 2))
 (segment (start 123 85.5) (end 122 84.5) (width 0.25) (layer "F.Cu") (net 9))
 (segment (start 124.075 96.425) (end 124.075 88.075) (width 0.25) (layer "F.Cu") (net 9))
 (segment (start 123 97.5) (end 124.075 96.425) (width 0.25) (layer "F.Cu") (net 9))
 (segment (start 122 84.5) (end 122 70.5) (width 0.25) (layer "F.Cu") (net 9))
 (segment (start 124 88) (end 124 86.5) (width 0.25) (layer "F.Cu") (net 9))
 (segment (start 124 86.5) (end 123 85.5) (width 0.25) (layer "F.Cu") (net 9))
 (segment (start 122 70.5) (end 124 68.5) (width 0.25) (layer "F.Cu") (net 9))
 (segment (start 124.075 88.075) (end 124 88) (width 0.25) (layer "F.Cu") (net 9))
 (segment (start 150 69) (end 154.287 73.287) (width 0.25) (layer "B.Cu") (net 9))
 (segment (start 154.287 85.287) (end 157 88) (width 0.25) (layer "B.Cu") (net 9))
 (segment (start 157 88) (end 160.4 88) (width 0.25) (layer "B.Cu") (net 9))
 (segment (start 160.4 88) (end 163.83 91.43) (width 0.25) (layer "B.Cu") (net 9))
 (segment (start 124 69) (end 150 69) (width 0.25) (layer "B.Cu") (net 9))
 (segment (start 154.287 73.287) (end 154.287 85.287) (width 0.25) (layer "B.Cu") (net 9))
 (segment (start 142.5 65) (end 149 65) (width 0.25) (layer "F.Cu") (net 5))
 (segment (start 149 65) (end 150.66 66.66) (width 0.25) (layer "F.Cu") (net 5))
 (segment (start 140.493 60.007) (end 140.493 62.993) (width 0.25) (layer "F.Cu") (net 5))
 (segment (start 141 59.5) (end 140.493 60.007) (width 0.25) (layer "F.Cu") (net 5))
 (segment (start 150.66 60.66) (end 149.5 59.5) (width 0.25) (layer "F.Cu") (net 5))
 (segment (start 140.493 62.993) (end 142.5 65) (width 0.25) (layer "F.Cu") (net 5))
 (segment (start 150.66 66.66) (end 150.66 76.62) (width 0.25) (layer "F.Cu") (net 5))
 (segment (start 149.5 59.5) (end 141 59.5) (width 0.25) (layer "F.Cu") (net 5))
 (segment (start 150.66 76.62) (end 152.27 78.23) (width 0.25) (layer "B.Cu") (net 5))
 (segment (start 152.27 78.23) (end 152.27 83.36) (width 0.25) (layer "B.Cu") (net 5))
 (segment (start 164.58 61.26) (end 164.58 76.5) (width 0.25) (layer "B.Cu") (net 7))
 (segment (start 164.58 76.5) (end 165.77 77.69) (width 0.25) (layer "B.Cu") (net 7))
 (segment (start 165.77 77.69) (end 165.77 83.22) (width 0.25) (layer "B.Cu") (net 7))
 (segment (start 169.66 61.26) (end 170.747 62.347) (width 0.25) (layer "F.Cu") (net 13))
 (segment (start 168 64.5) (end 169.66 62.84) (width 0.25) (layer "F.Cu") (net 13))
 (segment (start 170.747 95.622009) (end 160 106.369009) (width 0.25) (layer "F.Cu") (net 13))
 (segment (start 155.74 63.24) (end 157 64.5) (width 0.25) (layer "F.Cu") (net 13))
 (segment (start 143 64.5) (end 154.5 64.5) (width 0.25) (layer "F.Cu") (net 13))
 (segment (start 169.66 62.84) (end 169.66 61.26) (width 0.25) (layer "F.Cu") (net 13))
 (segment (start 157 64.5) (end 168 64.5) (width 0.25) (layer "F.Cu") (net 13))
 (segment (start 141.58 61.38) (end 141.58 63.08) (width 0.25) (layer "F.Cu") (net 13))
 (segment (start 155.74 63.26) (end 155.74 61.38) (width 0.25) (layer "F.Cu") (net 13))
 (segment (start 155.74 63.26) (end 155.74 63.24) (width 0.25) (layer "F.Cu") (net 13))
 (segment (start 142.8 108.5) (end 140.97 106.67) (width 0.25) (layer "F.Cu") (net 13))
 (segment (start 160 106.369009) (end 160 107.010991) (width 0.25) (layer "F.Cu") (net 13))
 (segment (start 141.58 63.08) (end 143 64.5) (width 0.25) (layer "F.Cu") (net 13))
 (segment (start 158.510991 108.5) (end 142.8 108.5) (width 0.25) (layer "F.Cu") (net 13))
 (segment (start 154.5 64.5) (end 155.74 63.26) (width 0.25) (layer "F.Cu") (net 13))
 (segment (start 160 107.010991) (end 158.510991 108.5) (width 0.25) (layer "F.Cu") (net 13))
 (segment (start 170.747 62.347) (end 170.747 95.622009) (width 0.25) (layer "F.Cu") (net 13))
 (segment (start 139.04 61.38) (end 139.04 59.46) (width 0.25) (layer "F.Cu") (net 14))
 (segment (start 141.34 104.5) (end 143.51 106.67) (width 0.25) (layer "F.Cu") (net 14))
 (segment (start 151.5 58) (end 153.2 59.7) (width 0.25) (layer "F.Cu") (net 14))
 (segment (start 165.5 58) (end 167.12 59.62) (width 0.25) (layer "F.Cu") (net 14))
 (segment (start 128.5 58.5) (end 128.5 101.5) (width 0.25) (layer "F.Cu") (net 14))
 (segment (start 139.04 61.38) (end 139.04 59.54) (width 0.25) (layer "F.Cu") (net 14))
 (segment (start 153.2 59.7) (end 153.2 61.38) (width 0.25) (layer "F.Cu") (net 14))
 (segment (start 131.5 104.5) (end 141.34 104.5) (width 0.25) (layer "F.Cu") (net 14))
 (segment (start 139.04 59.54) (end 137.5 58) (width 0.25) (layer "F.Cu") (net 14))
 (segment (start 129 58) (end 128.5 58.5) (width 0.25) (layer "F.Cu") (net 14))
 (segment (start 167.12 59.62) (end 167.12 61.26) (width 0.25) (layer "F.Cu") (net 14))
 (segment (start 128.5 101.5) (end 131.5 104.5) (width 0.25) (layer "F.Cu") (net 14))
 (segment (start 155 58) (end 165.5 58) (width 0.25) (layer "F.Cu") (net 14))
 (segment (start 153.3 59.7) (end 153.2 59.7) (width 0.25) (layer "F.Cu") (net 14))
 (segment (start 155 58) (end 153.3 59.7) (width 0.25) (layer "F.Cu") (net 14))
 (segment (start 139.04 59.46) (end 140.5 58) (width 0.25) (layer "F.Cu") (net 14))
 (segment (start 140.5 58) (end 151.5 58) (width 0.25) (layer "F.Cu") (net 14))
 (segment (start 137.5 58) (end 129 58) (width 0.25) (layer "F.Cu") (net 14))
 (segment (start 150 101) (end 158.5 101) (width 0.25) (layer "F.Cu") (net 15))
 (segment (start 146.05 106.67) (end 146.05 104.95) (width 0.25) (layer "F.Cu") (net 15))
 (segment (start 146.05 104.95) (end 150 101) (width 0.25) (layer "F.Cu") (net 15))
 (via (at 158.5 101) (size 0.8) (drill 0.4) (layers "F.Cu" "B.Cu") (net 15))
 (segment (start 149.5 64.5) (end 160.5 64.5) (width 0.25) (layer "B.Cu") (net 15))
 (segment (start 157.5 73.5) (end 157.5 81) (width 0.25) (layer "B.Cu") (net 15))
 (segment (start 165.245 94.255) (end 158.5 101) (width 0.25) (layer "B.Cu") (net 15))
 (segment (start 133.96 61.38) (end 133.96 62.96) (width 0.25) (layer "B.Cu") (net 15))
 (segment (start 160.5 64.5) (end 162.04 62.96) (width 0.25) (layer "B.Cu") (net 15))
 (segment (start 133.96 62.96) (end 135.5 64.5) (width 0.25) (layer "B.Cu") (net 15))
 (segment (start 165.245 88.745) (end 165.245 94.255) (width 0.25) (layer "B.Cu") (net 15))
 (segment (start 148.12 61.38) (end 148.12 63.12) (width 0.25) (layer "B.Cu") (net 15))
 (segment (start 157.5 81) (end 165.245 88.745) (width 0.25) (layer "B.Cu") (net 15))
 (segment (start 148.12 62.88) (end 148.12 61.38) (width 0.25) (layer "B.Cu") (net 15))
 (segment (start 148.12 63.12) (end 149.5 64.5) (width 0.25) (layer "B.Cu") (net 15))
 (segment (start 148.12 61.38) (end 148.12 64.12) (width 0.25) (layer "B.Cu") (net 15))
 (segment (start 162.04 62.96) (end 162.04 61.26) (width 0.25) (layer "B.Cu") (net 15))
 (segment (start 146.5 64.5) (end 148.12 62.88) (width 0.25) (layer "B.Cu") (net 15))
 (segment (start 135.5 64.5) (end 146.5 64.5) (width 0.25) (layer "B.Cu") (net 15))
 (segment (start 148.12 64.12) (end 157.5 73.5) (width 0.25) (layer "B.Cu") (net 15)))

